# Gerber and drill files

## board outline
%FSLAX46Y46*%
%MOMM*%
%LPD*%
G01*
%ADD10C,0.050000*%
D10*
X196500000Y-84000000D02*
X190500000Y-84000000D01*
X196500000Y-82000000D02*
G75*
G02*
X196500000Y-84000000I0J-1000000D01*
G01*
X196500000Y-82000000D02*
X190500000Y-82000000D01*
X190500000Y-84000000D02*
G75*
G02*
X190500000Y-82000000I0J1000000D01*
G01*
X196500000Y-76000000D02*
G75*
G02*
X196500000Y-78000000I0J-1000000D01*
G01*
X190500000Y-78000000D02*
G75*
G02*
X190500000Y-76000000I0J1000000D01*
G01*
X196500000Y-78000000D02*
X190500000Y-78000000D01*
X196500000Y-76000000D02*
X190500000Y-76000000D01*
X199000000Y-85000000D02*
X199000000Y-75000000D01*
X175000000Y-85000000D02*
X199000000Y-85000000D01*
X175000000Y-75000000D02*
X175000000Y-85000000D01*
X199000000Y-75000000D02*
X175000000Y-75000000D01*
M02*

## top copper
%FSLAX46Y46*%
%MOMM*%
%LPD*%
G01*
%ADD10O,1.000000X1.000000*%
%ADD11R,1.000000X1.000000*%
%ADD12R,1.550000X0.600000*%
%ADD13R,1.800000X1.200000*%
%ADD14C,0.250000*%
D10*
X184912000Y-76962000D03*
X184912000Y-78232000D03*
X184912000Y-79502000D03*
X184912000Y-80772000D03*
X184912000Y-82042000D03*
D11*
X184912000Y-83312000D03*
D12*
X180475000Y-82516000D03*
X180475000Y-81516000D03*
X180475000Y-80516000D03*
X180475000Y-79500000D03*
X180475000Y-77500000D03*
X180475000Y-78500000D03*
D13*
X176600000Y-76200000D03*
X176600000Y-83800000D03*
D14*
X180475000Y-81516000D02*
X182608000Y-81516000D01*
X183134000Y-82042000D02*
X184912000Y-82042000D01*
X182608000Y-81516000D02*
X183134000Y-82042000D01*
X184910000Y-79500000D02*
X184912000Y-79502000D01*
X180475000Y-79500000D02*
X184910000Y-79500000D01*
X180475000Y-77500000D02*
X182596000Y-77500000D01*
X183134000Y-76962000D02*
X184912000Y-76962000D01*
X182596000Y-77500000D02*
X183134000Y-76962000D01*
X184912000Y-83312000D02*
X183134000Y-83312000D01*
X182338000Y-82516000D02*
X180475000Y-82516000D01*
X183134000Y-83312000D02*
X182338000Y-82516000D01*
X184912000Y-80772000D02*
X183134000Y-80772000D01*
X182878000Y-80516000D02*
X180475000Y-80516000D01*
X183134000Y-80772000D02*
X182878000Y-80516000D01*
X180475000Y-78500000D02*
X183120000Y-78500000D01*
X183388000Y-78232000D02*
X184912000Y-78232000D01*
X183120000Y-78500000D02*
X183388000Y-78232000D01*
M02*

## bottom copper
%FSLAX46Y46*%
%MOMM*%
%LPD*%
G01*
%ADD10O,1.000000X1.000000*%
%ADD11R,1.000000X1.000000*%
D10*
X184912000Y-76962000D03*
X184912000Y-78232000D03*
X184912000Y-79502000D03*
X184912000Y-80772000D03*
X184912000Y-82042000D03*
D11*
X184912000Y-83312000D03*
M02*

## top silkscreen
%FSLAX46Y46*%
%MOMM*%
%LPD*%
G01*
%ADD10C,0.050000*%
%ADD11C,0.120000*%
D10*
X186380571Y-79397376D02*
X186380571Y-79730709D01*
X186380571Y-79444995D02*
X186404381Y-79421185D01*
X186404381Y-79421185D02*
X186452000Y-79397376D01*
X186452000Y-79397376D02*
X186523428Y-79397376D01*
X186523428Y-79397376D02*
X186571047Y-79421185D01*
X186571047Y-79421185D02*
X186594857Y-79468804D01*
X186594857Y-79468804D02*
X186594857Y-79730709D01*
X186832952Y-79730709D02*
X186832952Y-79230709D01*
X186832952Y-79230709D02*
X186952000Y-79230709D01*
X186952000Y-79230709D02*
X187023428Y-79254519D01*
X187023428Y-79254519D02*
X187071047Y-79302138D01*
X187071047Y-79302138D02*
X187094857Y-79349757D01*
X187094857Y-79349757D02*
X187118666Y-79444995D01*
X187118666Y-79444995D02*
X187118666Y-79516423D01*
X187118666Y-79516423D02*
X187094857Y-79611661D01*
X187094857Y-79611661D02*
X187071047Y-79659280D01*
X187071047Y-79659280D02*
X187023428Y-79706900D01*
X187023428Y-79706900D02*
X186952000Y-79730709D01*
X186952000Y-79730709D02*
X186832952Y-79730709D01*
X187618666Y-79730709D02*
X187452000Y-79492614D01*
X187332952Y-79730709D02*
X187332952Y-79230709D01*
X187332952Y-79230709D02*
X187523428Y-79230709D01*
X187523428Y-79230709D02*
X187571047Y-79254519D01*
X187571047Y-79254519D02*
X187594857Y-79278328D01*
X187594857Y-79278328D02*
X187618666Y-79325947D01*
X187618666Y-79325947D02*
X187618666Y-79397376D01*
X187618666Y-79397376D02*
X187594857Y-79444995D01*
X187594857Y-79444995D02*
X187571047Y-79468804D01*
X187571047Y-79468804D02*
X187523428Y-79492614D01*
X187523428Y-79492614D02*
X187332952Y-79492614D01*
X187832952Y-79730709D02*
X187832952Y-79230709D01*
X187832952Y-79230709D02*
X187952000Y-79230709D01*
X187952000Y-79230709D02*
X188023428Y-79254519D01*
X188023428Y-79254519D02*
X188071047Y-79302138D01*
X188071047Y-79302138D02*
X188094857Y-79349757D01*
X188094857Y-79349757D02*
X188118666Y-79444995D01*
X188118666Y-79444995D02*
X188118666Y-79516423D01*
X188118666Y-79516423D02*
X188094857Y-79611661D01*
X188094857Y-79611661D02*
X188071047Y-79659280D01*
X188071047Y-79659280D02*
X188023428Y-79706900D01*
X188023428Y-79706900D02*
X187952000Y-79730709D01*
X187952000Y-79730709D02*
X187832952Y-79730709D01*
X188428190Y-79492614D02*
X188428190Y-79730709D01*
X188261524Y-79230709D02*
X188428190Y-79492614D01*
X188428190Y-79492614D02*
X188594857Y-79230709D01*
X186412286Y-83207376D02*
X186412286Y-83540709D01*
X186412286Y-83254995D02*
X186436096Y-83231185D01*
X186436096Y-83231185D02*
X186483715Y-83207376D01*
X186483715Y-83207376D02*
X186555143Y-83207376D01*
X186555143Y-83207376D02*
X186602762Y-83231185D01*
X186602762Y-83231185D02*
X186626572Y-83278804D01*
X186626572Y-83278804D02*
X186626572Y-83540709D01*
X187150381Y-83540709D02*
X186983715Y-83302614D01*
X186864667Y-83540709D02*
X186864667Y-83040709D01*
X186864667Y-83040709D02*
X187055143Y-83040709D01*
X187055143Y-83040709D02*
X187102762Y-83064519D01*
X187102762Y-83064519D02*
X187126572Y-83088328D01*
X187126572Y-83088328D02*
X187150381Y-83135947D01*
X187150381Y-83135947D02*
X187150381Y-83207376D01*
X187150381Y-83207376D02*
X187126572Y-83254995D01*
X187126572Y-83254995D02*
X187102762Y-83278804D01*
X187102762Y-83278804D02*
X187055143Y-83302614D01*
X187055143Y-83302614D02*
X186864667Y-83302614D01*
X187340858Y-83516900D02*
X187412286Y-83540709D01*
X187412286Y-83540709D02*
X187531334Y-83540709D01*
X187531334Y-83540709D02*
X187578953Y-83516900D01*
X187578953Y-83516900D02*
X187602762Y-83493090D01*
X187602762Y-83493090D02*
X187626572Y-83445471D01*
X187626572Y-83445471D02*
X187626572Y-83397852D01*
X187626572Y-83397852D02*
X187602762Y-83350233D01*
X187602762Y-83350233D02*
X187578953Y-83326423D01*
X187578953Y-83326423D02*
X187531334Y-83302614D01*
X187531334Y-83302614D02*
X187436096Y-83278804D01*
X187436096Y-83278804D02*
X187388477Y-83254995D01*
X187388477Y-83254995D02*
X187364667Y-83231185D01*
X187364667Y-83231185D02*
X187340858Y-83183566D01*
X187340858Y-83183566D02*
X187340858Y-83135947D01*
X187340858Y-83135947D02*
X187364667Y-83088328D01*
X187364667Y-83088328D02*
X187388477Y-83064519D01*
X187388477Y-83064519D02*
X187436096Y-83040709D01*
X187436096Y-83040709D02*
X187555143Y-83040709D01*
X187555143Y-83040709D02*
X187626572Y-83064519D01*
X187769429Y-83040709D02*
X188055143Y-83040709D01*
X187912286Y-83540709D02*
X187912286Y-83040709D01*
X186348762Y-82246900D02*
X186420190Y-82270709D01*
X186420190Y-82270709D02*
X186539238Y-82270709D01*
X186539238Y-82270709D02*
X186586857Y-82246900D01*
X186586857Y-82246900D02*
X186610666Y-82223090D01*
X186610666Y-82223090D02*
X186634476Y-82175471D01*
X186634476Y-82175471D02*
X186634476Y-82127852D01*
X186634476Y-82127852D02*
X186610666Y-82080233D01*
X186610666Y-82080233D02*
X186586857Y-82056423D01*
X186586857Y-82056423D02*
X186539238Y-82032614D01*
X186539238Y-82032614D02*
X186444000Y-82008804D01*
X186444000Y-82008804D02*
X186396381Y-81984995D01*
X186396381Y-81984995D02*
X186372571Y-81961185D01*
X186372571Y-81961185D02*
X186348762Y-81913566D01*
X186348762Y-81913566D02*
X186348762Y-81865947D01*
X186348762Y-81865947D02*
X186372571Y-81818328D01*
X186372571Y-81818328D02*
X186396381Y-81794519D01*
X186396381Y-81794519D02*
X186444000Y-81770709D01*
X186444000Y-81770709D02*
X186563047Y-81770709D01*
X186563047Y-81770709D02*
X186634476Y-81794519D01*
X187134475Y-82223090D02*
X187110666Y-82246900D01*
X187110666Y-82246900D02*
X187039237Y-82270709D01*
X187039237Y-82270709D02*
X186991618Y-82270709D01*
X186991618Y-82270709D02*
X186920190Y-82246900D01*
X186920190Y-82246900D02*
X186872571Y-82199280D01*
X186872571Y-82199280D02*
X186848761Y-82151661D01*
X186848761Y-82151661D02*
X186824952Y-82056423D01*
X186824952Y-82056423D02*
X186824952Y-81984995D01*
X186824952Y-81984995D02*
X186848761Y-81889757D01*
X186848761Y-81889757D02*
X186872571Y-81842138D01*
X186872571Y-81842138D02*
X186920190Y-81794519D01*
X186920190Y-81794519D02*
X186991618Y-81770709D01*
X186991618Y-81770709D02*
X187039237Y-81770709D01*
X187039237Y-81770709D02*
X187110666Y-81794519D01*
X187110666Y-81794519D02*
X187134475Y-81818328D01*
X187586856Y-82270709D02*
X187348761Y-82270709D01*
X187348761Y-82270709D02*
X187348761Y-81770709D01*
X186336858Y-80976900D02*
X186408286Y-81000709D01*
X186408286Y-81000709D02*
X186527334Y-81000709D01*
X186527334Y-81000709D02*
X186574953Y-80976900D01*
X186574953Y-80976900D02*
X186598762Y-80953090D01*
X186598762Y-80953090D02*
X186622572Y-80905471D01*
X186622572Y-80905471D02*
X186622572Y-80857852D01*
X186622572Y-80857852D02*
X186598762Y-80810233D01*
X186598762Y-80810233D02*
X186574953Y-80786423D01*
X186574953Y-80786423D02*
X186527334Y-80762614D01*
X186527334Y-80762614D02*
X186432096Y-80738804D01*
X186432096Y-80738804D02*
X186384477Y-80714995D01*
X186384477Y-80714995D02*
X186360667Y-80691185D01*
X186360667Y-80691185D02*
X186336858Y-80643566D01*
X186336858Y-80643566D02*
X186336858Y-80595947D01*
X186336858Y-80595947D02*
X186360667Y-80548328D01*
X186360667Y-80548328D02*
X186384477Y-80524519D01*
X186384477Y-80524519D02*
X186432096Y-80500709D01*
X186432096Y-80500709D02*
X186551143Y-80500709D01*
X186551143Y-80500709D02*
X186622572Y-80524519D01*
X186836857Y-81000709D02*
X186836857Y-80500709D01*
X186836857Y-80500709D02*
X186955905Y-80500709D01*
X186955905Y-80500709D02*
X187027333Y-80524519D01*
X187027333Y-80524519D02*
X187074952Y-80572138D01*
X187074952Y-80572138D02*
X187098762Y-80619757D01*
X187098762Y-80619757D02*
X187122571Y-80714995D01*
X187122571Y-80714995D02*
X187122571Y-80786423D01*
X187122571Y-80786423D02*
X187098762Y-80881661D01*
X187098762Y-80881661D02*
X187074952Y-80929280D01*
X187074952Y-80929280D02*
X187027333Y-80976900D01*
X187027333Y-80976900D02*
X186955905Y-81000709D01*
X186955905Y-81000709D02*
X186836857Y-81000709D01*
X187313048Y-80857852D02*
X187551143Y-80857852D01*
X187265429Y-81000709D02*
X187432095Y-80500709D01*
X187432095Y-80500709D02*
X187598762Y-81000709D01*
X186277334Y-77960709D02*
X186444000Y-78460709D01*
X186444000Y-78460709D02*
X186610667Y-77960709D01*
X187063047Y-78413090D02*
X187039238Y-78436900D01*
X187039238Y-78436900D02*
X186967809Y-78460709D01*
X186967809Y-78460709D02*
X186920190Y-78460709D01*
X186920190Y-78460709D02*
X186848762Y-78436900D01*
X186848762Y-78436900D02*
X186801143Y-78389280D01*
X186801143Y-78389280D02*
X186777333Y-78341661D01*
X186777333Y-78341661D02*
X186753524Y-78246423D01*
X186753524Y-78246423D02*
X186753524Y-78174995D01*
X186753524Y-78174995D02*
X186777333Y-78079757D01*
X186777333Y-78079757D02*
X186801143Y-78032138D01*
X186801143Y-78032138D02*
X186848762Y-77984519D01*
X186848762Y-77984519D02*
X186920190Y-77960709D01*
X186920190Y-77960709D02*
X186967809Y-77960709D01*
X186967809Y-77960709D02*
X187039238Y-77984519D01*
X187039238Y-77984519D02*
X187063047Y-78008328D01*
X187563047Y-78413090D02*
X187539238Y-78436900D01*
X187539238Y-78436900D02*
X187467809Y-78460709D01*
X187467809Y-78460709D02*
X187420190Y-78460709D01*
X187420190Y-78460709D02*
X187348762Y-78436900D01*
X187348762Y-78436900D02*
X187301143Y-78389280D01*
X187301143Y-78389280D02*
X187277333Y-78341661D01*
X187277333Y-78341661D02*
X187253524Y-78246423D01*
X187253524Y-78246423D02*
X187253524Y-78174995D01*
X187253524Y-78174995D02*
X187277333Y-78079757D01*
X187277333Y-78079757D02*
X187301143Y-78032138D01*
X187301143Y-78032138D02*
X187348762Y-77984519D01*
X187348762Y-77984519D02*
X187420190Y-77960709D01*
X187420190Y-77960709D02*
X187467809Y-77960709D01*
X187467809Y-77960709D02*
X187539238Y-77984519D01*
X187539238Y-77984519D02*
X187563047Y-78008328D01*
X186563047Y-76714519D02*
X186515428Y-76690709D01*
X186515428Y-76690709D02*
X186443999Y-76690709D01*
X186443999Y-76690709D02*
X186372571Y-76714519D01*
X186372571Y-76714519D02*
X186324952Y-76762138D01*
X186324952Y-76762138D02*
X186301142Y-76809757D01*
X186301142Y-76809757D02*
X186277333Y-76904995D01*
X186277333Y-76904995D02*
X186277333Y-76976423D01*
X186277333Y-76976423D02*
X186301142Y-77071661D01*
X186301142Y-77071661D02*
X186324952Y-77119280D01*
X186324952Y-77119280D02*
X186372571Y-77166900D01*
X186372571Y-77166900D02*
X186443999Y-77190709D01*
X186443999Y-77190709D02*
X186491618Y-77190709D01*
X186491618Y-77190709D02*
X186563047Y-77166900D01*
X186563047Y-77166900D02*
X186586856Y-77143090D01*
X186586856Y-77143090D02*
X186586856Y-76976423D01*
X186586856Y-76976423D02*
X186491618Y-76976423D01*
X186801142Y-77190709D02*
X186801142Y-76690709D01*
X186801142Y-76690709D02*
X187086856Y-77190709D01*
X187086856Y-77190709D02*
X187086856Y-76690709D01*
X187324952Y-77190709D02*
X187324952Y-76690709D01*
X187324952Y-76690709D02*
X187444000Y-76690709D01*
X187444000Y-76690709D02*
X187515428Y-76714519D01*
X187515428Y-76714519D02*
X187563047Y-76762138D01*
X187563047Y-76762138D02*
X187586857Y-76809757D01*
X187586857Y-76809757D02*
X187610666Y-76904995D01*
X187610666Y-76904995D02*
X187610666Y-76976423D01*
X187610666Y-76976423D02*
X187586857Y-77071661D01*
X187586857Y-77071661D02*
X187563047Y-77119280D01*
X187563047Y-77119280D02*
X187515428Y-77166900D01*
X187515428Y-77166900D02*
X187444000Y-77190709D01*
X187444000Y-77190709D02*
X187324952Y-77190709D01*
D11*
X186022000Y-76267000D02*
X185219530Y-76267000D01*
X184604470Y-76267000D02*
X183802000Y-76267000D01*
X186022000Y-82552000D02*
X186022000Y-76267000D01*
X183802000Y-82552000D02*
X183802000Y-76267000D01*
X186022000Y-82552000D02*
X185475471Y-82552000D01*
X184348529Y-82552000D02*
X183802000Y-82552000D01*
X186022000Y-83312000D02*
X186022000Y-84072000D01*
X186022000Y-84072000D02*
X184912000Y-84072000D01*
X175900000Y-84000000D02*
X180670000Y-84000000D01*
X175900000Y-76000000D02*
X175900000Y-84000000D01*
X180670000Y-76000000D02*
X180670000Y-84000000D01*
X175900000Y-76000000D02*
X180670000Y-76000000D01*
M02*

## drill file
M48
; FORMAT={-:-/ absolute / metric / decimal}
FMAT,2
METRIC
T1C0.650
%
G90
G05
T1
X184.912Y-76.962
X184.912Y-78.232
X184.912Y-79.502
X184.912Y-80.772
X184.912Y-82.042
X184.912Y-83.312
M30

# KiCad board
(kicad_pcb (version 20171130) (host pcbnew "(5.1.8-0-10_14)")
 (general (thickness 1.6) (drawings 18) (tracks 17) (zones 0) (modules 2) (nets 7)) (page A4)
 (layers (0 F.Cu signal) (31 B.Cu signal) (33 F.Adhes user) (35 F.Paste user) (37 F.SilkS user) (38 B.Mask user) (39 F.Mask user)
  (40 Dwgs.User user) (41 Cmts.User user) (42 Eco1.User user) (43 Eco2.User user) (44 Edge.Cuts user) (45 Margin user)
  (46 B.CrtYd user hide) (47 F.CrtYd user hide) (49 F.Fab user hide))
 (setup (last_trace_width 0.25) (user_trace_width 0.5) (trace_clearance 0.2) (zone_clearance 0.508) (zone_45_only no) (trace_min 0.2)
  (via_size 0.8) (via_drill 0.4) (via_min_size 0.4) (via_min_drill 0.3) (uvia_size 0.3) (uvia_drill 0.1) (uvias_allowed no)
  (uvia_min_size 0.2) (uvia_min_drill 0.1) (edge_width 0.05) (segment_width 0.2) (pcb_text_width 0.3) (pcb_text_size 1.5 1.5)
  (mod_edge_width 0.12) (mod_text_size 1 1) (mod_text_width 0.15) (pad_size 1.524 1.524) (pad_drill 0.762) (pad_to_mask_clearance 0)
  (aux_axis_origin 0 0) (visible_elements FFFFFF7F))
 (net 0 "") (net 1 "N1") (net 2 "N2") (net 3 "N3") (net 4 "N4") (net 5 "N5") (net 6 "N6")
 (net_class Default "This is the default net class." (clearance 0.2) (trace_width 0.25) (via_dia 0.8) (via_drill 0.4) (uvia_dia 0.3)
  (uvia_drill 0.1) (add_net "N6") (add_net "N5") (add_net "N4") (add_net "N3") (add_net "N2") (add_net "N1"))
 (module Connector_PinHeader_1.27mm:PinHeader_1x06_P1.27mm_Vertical (layer F.Cu) (at 184.912 83.312 180)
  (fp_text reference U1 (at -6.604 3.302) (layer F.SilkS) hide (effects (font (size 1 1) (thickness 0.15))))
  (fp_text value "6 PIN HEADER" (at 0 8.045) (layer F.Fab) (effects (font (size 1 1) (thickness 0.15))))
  (fp_line (start -1.11 7.045) (end -0.30753 7.045) (layer F.SilkS) (width 0.12))
  (fp_line (start 0.30753 7.045) (end 1.11 7.045) (layer F.SilkS) (width 0.12))
  (fp_line (start -1.11 0.76) (end -1.11 7.045) (layer F.SilkS) (width 0.12))
  (fp_line (start 1.11 0.76) (end 1.11 7.045) (layer F.SilkS) (width 0.12))
  (fp_line (start -1.11 0.76) (end -0.563471 0.76) (layer F.SilkS) (width 0.12))
  (fp_line (start 0.563471 0.76) (end 1.11 0.76) (layer F.SilkS) (width 0.12))
  (fp_line (start -1.11 0) (end -1.11 -0.76) (layer F.SilkS) (width 0.12))
  (fp_line (start -1.11 -0.76) (end 0 -0.76) (layer F.SilkS) (width 0.12))
  (pad 6 thru_hole oval (at 0 6.35 180) (size 1 1) (drill 0.65) (layers *.Cu *.Mask) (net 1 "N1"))
  (pad 5 thru_hole oval (at 0 5.08 180) (size 1 1) (drill 0.65) (layers *.Cu *.Mask) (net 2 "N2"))
  (pad 4 thru_hole oval (at 0 3.81 180) (size 1 1) (drill 0.65) (layers *.Cu *.Mask) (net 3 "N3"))
  (pad 3 thru_hole oval (at 0 2.54 180) (size 1 1) (drill 0.65) (layers *.Cu *.Mask) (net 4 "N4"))
  (pad 2 thru_hole oval (at 0 1.27 180) (size 1 1) (drill 0.65) (layers *.Cu *.Mask) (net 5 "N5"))
  (pad 1 thru_hole rect (at 0 0 180) (size 1 1) (drill 0.65) (layers *.Cu *.Mask) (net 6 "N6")))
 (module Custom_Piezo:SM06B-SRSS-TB (layer F.Cu) (at 176.6 80 270)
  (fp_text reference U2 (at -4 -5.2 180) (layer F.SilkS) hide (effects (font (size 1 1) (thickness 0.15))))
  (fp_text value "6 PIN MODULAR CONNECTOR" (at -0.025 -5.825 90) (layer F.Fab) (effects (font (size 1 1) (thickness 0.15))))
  (fp_line (start 4 0.7) (end 4 -4.07) (layer F.SilkS) (width 0.12))
  (fp_line (start -4 0.7) (end 4 0.7) (layer F.SilkS) (width 0.12))
  (fp_line (start -4 -4.07) (end 4 -4.07) (layer F.SilkS) (width 0.12))
  (fp_line (start -4 0.7) (end -4 -4.07) (layer F.SilkS) (width 0.12))
  (pad 6 smd rect (at 2.516 -3.875 270) (size 0.6 1.55) (layers F.Cu F.Paste F.Mask) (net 6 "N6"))
  (pad 5 smd rect (at 1.516 -3.875 270) (size 0.6 1.55) (layers F.Cu F.Paste F.Mask) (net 5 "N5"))
  (pad 4 smd rect (at 0.516 -3.875 270) (size 0.6 1.55) (layers F.Cu F.Paste F.Mask) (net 4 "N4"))
  (pad 3 smd rect (at -0.5 -3.875 270) (size 0.6 1.55) (layers F.Cu F.Paste F.Mask) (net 3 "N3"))
  (pad 1 smd rect (at -2.5 -3.875 270) (size 0.6 1.55) (layers F.Cu F.Paste F.Mask) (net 1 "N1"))
  (pad 2 smd rect (at -1.5 -3.875 270) (size 0.6 1.55) (layers F.Cu F.Paste F.Mask) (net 2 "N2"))
  (pad "" smd rect (at -3.8 0 270) (size 1.2 1.8) (layers F.Cu F.Paste F.Mask))
  (pad "" smd rect (at 3.8 0 270) (size 1.2 1.8) (layers F.Cu F.Paste F.Mask)))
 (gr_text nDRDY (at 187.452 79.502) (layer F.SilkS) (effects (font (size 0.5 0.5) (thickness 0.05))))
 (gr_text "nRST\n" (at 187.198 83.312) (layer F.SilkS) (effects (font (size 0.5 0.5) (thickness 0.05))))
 (gr_line (start 196.5 84) (end 190.5 84) (layer Edge.Cuts) (width 0.05))
 (gr_arc (start 196.5 83) (end 196.5 84) (angle -180) (layer Edge.Cuts) (width 0.05))
 (gr_line (start 196.5 82) (end 190.5 82) (layer Edge.Cuts) (width 0.05))
 (gr_arc (start 190.5 83) (end 190.5 82) (angle -180) (layer Edge.Cuts) (width 0.05))
 (gr_arc (start 196.5 77) (end 196.5 78) (angle -180) (layer Edge.Cuts) (width 0.05))
 (gr_arc (start 190.5 77) (end 190.5 76) (angle -180) (layer Edge.Cuts) (width 0.05))
 (gr_line (start 196.5 78) (end 190.5 78) (layer Edge.Cuts) (width 0.05))
 (gr_line (start 196.5 76) (end 190.5 76) (layer Edge.Cuts) (width 0.05))
 (gr_line (start 199 85) (end 199 75) (layer Edge.Cuts) (width 0.05))
 (gr_line (start 175 85) (end 199 85) (layer Edge.Cuts) (width 0.05))
 (gr_line (start 175 75) (end 175 85) (layer Edge.Cuts) (width 0.05))
 (gr_line (start 199 75) (end 175 75) (layer Edge.Cuts) (width 0.05))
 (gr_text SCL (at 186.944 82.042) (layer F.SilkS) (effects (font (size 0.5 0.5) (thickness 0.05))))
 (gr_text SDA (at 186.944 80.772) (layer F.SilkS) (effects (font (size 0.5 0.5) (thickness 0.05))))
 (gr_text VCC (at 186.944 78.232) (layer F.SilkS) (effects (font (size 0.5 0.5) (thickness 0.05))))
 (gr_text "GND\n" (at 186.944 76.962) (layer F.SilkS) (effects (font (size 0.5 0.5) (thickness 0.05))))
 (segment (start 180.475 81.516) (end 182.608 81.516) (width 0.25) (layer F.Cu) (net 5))
 (segment (start 183.134 82.042) (end 184.912 82.042) (width 0.25) (layer F.Cu) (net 5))
 (segment (start 182.608 81.516) (end 183.134 82.042) (width 0.25) (layer F.Cu) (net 5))
 (segment (start 184.91 79.5) (end 184.912 79.502) (width 0.25) (layer F.Cu) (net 3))
 (segment (start 180.475 79.5) (end 184.91 79.5) (width 0.25) (layer F.Cu) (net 3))
 (segment (start 180.475 77.5) (end 182.596 77.5) (width 0.25) (layer F.Cu) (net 1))
 (segment (start 183.134 76.962) (end 184.912 76.962) (width 0.25) (layer F.Cu) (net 1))
 (segment (start 182.596 77.5) (end 183.134 76.962) (width 0.25) (layer F.Cu) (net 1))
 (segment (start 184.912 83.312) (end 183.134 83.312) (width 0.25) (layer F.Cu) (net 6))
 (segment (start 182.338 82.516) (end 180.475 82.516) (width 0.25) (layer F.Cu) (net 6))
 (segment (start 183.134 83.312) (end 182.338 82.516) (width 0.25) (layer F.Cu) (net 6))
 (segment (start 184.912 80.772) (end 183.134 80.772) (width 0.25) (layer F.Cu) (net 4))
 (segment (start 182.878 80.516) (end 180.475 80.516) (width 0.25) (layer F.Cu) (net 4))
 (segment (start 183.134 80.772) (end 182.878 80.516) (width 0.25) (layer F.Cu) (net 4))
 (segment (start 180.475 78.5) (end 183.12 78.5) (width 0.25) (layer F.Cu) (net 2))
 (segment (start 183.388 78.232) (end 184.912 78.232) (width 0.25) (layer F.Cu) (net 2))
 (segment (start 183.12 78.5) (end 183.388 78.232) (width 0.25) (layer F.Cu) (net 2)))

